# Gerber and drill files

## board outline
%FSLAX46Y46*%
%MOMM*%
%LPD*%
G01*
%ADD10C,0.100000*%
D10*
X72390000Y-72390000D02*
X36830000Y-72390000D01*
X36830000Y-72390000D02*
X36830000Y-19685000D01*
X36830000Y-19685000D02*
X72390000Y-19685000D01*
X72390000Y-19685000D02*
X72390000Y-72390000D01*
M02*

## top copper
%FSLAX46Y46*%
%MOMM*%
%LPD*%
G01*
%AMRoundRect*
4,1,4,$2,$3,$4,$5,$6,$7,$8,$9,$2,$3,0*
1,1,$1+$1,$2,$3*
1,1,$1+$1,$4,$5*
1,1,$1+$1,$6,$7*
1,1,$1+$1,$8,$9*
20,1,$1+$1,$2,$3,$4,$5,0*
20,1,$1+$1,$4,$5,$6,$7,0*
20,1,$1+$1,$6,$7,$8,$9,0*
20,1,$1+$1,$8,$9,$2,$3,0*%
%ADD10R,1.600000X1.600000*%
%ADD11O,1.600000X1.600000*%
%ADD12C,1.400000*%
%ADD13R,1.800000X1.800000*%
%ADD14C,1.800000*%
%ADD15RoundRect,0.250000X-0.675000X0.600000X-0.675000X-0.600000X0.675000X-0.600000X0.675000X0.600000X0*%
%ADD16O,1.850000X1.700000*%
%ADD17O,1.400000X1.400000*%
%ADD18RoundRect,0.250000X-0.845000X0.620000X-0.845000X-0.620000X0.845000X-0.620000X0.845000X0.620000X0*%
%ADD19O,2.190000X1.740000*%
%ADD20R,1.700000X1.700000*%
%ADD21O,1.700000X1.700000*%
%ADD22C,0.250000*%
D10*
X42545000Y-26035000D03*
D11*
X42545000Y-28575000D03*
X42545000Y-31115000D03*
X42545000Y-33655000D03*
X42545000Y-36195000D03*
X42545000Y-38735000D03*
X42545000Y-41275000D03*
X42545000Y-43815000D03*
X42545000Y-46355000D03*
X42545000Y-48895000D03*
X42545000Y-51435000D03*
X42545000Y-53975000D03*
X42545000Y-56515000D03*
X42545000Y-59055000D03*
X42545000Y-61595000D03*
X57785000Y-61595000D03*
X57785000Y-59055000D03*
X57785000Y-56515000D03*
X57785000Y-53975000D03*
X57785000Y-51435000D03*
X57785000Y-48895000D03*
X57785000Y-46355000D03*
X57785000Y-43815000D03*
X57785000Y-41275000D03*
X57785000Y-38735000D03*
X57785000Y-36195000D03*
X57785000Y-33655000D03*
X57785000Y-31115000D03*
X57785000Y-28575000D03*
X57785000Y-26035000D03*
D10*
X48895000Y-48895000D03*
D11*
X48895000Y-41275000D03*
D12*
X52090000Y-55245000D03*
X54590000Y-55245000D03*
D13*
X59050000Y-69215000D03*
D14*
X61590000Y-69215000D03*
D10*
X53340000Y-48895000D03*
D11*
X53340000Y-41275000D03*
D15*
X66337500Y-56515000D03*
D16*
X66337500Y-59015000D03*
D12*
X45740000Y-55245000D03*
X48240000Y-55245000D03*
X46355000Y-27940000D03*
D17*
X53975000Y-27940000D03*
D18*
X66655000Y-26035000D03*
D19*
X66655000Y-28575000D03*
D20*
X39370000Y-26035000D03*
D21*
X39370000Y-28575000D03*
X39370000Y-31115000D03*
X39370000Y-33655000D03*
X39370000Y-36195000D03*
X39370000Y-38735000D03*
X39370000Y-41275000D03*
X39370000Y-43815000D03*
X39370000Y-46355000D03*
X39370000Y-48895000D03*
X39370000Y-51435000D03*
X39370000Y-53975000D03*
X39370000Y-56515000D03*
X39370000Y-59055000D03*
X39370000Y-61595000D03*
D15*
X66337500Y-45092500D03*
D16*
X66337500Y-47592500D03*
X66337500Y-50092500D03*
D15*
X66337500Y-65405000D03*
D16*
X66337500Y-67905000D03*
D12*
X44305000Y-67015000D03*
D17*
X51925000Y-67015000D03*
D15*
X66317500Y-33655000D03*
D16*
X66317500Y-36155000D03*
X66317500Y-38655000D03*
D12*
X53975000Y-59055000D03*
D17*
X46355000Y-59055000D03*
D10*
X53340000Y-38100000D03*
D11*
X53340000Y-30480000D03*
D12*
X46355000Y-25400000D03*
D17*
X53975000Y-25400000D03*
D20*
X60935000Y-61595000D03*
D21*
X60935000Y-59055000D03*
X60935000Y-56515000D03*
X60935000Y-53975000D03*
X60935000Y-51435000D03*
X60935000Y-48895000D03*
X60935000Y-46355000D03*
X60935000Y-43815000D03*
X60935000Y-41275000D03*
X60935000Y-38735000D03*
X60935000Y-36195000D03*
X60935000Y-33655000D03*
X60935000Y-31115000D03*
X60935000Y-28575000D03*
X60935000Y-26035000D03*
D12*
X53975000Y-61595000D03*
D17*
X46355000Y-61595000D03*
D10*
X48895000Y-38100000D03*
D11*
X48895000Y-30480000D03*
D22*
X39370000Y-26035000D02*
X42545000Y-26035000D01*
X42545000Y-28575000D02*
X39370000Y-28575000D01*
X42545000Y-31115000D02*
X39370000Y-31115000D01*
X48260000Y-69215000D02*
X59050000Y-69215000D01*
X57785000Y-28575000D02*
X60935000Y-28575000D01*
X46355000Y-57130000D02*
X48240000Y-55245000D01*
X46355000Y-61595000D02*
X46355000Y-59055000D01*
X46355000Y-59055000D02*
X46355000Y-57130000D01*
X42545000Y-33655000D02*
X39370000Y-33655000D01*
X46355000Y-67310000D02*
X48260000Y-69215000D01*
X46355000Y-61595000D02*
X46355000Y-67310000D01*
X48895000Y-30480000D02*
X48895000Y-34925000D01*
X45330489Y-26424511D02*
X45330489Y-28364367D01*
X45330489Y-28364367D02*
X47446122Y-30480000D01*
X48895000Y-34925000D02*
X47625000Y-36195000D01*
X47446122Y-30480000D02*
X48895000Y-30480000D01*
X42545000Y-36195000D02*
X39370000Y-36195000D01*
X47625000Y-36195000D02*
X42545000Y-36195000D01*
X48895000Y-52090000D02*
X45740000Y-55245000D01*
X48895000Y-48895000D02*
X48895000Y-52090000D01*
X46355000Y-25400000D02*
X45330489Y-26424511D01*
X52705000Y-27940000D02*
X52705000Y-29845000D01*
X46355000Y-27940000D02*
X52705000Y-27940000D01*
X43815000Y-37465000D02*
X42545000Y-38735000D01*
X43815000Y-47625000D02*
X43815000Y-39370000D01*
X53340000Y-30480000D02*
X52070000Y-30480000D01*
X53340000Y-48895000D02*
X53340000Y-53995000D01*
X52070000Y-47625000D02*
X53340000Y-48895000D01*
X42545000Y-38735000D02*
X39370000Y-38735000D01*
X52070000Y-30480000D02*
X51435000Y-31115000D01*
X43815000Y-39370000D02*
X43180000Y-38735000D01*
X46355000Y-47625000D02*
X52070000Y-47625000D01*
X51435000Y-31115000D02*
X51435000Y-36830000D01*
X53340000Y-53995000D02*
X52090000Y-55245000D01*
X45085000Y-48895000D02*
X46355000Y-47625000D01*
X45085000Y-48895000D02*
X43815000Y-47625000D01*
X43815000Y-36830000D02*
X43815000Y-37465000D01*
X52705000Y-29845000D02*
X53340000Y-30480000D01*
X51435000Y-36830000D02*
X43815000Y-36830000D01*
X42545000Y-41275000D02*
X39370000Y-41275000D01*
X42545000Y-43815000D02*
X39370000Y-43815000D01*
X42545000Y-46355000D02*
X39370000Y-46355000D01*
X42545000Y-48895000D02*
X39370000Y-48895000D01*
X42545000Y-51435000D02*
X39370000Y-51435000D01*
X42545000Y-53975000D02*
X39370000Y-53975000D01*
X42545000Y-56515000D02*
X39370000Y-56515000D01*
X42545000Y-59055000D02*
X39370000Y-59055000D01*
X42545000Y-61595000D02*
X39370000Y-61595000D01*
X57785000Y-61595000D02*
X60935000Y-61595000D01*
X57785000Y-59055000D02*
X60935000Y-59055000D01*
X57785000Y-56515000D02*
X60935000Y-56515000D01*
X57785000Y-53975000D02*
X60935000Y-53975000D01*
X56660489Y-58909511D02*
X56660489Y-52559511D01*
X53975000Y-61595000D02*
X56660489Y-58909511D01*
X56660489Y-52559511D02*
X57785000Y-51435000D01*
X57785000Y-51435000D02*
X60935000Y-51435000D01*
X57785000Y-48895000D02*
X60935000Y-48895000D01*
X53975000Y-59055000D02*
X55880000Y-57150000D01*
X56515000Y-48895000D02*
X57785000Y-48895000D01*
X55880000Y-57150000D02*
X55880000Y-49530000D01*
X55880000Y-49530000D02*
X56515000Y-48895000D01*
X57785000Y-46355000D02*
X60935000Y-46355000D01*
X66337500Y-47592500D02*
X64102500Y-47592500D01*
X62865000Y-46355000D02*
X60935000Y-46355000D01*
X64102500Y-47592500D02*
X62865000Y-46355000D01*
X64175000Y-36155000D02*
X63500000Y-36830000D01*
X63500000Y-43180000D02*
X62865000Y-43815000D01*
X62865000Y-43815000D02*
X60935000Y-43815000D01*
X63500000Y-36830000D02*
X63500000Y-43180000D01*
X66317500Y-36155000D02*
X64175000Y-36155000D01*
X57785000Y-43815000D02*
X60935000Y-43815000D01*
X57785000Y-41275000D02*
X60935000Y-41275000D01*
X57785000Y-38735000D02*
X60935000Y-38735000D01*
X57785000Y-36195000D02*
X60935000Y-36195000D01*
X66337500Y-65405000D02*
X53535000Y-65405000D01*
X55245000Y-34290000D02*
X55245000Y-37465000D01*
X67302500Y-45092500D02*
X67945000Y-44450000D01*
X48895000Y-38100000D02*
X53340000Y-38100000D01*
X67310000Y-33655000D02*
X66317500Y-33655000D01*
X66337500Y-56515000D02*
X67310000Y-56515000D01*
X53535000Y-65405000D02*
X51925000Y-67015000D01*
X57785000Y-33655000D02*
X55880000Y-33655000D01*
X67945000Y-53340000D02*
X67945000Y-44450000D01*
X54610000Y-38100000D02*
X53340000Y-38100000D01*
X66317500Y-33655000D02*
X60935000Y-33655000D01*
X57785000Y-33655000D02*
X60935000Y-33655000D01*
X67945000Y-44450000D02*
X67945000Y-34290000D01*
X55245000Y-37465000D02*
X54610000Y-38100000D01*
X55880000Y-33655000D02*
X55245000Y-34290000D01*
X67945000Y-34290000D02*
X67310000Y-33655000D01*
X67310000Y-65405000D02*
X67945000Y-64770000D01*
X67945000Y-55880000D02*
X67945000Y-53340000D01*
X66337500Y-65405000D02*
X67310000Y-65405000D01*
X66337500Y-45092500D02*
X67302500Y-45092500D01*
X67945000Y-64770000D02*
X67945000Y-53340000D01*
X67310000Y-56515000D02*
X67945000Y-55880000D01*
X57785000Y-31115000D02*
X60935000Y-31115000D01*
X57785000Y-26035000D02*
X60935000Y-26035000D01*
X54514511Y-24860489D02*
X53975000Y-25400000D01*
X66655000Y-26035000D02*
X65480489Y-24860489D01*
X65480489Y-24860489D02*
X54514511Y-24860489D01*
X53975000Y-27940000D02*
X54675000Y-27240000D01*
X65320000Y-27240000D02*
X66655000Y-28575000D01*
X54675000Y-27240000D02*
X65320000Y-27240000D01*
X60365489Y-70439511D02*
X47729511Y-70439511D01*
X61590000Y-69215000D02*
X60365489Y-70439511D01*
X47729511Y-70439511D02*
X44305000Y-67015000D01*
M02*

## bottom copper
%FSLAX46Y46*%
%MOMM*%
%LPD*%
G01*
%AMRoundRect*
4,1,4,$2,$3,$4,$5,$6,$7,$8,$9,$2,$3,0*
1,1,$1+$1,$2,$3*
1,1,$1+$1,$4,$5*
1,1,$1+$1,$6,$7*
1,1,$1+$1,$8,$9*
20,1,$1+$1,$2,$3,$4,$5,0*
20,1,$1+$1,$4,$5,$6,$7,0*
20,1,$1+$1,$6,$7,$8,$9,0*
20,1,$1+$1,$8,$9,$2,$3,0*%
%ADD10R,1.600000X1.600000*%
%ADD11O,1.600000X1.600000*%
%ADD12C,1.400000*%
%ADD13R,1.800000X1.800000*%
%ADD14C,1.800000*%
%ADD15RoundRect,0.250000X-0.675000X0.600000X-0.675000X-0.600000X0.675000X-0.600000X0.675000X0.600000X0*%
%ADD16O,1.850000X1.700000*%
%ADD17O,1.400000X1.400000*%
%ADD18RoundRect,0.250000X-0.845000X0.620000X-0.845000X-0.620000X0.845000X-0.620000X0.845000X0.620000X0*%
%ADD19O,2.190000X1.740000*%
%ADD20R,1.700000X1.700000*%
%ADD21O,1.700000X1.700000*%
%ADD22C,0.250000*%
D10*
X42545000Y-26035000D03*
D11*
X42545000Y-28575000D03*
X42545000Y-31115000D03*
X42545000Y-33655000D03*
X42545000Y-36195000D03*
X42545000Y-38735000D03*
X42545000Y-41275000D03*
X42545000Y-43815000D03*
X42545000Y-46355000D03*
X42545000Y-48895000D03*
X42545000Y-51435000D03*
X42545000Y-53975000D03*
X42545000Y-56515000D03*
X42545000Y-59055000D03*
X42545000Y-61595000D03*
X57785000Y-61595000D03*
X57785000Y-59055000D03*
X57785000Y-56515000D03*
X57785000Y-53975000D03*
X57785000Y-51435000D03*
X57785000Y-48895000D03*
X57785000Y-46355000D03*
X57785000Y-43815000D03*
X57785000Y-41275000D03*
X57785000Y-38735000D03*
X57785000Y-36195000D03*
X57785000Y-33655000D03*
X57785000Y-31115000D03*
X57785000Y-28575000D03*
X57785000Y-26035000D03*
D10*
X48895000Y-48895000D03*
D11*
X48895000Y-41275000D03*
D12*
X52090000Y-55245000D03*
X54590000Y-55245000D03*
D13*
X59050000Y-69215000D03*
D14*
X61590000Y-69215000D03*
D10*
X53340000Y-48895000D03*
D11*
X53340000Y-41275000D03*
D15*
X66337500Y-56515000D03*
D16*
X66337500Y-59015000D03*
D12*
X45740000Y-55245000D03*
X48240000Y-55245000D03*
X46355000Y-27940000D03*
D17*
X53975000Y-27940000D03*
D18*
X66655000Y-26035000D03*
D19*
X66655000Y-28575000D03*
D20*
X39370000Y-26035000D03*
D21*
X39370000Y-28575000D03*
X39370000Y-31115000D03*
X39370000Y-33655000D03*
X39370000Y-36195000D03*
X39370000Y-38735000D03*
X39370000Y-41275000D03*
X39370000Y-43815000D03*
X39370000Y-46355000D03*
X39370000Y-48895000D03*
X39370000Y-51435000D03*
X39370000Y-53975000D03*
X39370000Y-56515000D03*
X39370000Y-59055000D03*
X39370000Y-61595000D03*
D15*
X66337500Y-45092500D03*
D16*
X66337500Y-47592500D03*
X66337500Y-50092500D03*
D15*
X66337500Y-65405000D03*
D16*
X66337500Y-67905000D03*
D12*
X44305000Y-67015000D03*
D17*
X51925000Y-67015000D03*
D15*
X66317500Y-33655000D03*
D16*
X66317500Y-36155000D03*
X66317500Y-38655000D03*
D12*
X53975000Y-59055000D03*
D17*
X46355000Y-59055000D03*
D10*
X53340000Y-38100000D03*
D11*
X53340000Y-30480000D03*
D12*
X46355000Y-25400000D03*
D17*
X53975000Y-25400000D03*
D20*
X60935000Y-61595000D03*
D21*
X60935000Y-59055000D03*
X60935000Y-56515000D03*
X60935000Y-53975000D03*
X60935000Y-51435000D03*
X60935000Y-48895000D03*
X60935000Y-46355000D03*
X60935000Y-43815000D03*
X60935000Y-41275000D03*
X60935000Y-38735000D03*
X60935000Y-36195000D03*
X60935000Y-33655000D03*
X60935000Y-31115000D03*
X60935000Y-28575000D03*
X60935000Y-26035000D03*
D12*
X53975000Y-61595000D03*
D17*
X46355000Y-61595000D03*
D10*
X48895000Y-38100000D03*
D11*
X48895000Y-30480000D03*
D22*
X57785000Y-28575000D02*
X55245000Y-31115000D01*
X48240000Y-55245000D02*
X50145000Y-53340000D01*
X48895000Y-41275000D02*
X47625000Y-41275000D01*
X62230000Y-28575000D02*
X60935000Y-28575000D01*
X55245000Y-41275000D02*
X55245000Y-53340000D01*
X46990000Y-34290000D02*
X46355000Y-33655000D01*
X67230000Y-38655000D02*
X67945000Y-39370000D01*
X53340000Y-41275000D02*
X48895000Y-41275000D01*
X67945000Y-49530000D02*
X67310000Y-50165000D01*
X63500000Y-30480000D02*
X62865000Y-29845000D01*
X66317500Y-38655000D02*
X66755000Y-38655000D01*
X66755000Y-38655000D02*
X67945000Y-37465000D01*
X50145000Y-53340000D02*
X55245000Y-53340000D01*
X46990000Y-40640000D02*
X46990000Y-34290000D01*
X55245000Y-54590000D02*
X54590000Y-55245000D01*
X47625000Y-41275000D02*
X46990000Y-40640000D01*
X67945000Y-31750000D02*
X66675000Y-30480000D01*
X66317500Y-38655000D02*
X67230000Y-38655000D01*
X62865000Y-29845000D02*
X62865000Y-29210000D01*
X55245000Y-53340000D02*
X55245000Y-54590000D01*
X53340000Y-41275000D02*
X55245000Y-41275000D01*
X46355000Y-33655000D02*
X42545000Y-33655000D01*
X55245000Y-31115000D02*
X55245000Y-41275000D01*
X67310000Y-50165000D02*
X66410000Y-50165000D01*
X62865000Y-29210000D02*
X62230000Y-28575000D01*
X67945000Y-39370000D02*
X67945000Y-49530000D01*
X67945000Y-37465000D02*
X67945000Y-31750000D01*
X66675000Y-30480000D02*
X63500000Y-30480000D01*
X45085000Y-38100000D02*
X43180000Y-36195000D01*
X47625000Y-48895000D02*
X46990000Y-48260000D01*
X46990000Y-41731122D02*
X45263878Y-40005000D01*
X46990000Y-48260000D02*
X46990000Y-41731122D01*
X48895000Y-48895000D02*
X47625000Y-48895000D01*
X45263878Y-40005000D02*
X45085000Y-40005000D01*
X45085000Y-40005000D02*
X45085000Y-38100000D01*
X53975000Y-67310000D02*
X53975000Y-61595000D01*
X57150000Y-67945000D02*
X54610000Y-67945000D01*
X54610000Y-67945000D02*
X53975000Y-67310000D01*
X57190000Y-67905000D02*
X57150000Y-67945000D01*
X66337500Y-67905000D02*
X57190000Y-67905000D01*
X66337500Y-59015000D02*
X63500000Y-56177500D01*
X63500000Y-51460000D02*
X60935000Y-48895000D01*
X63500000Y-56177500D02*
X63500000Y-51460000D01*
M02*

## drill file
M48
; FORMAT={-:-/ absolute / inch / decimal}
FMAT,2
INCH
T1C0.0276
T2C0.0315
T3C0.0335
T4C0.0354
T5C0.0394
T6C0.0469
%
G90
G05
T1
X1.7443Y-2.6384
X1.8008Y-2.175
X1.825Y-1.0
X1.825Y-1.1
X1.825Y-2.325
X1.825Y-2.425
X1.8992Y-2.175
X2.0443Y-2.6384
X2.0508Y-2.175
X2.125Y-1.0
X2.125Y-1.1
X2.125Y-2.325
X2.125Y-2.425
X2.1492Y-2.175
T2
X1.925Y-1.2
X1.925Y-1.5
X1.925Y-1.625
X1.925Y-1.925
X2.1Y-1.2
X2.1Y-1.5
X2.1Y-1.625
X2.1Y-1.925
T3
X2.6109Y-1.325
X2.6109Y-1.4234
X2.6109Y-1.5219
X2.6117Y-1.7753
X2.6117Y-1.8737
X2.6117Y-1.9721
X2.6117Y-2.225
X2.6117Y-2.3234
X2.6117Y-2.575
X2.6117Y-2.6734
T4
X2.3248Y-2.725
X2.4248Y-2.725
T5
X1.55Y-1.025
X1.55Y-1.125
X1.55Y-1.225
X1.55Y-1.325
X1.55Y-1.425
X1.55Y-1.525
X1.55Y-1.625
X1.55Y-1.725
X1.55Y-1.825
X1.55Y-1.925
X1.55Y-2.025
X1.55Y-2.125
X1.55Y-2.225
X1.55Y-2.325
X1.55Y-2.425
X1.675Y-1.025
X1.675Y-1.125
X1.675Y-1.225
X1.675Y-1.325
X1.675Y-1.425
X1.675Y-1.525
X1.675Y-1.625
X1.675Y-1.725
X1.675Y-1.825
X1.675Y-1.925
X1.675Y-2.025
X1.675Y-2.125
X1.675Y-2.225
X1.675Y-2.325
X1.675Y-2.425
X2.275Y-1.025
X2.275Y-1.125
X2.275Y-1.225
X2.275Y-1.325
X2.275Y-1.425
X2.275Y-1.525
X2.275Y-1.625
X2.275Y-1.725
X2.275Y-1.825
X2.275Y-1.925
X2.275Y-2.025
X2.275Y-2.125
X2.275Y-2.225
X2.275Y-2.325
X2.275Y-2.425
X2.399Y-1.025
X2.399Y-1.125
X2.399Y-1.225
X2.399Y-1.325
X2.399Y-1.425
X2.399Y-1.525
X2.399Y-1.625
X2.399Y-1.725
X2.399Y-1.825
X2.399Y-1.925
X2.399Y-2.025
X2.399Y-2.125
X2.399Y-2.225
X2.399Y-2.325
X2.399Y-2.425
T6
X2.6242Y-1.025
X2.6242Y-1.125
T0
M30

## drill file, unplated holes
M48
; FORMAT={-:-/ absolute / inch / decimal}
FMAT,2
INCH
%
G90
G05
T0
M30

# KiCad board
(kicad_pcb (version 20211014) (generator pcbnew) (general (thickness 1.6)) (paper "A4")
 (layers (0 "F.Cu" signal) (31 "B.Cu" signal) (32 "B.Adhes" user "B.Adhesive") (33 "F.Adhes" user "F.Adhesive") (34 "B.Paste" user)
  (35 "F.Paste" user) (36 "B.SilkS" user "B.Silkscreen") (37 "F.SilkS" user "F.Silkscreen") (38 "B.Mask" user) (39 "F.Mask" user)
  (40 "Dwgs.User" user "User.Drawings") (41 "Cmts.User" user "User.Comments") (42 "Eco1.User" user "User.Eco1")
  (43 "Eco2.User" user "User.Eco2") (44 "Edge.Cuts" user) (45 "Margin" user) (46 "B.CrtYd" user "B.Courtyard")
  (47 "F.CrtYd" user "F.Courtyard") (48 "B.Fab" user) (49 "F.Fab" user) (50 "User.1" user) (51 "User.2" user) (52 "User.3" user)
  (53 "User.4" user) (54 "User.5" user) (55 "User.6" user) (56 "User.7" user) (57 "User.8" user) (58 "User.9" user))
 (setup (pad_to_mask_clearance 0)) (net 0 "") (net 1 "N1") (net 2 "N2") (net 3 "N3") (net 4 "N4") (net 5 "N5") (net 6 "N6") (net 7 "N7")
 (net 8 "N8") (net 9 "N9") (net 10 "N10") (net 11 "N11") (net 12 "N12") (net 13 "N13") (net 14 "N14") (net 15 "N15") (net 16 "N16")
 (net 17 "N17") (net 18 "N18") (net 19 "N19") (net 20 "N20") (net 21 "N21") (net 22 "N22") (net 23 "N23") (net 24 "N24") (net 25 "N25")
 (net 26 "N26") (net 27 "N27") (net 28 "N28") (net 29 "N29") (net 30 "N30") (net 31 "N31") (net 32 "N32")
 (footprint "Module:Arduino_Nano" (layer "F.Cu") (at 42.545 26.035)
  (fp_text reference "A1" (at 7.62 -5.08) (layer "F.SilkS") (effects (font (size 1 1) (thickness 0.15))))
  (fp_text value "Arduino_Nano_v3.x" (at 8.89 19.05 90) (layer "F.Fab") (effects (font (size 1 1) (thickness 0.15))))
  (pad "1" thru_hole rect (at 0 0) (size 1.6 1.6) (drill 1) (layers *.Cu *.Mask) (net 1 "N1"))
  (pad "2" thru_hole oval (at 0 2.54) (size 1.6 1.6) (drill 1) (layers *.Cu *.Mask) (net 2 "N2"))
  (pad "3" thru_hole oval (at 0 5.08) (size 1.6 1.6) (drill 1) (layers *.Cu *.Mask) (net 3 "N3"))
  (pad "4" thru_hole oval (at 0 7.62) (size 1.6 1.6) (drill 1) (layers *.Cu *.Mask) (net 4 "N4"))
  (pad "5" thru_hole oval (at 0 10.16) (size 1.6 1.6) (drill 1) (layers *.Cu *.Mask) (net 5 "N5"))
  (pad "6" thru_hole oval (at 0 12.7) (size 1.6 1.6) (drill 1) (layers *.Cu *.Mask) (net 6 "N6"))
  (pad "7" thru_hole oval (at 0 15.24) (size 1.6 1.6) (drill 1) (layers *.Cu *.Mask) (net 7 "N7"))
  (pad "8" thru_hole oval (at 0 17.78) (size 1.6 1.6) (drill 1) (layers *.Cu *.Mask) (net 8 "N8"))
  (pad "9" thru_hole oval (at 0 20.32) (size 1.6 1.6) (drill 1) (layers *.Cu *.Mask) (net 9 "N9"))
  (pad "10" thru_hole oval (at 0 22.86) (size 1.6 1.6) (drill 1) (layers *.Cu *.Mask) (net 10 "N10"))
  (pad "11" thru_hole oval (at 0 25.4) (size 1.6 1.6) (drill 1) (layers *.Cu *.Mask) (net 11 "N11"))
  (pad "12" thru_hole oval (at 0 27.94) (size 1.6 1.6) (drill 1) (layers *.Cu *.Mask) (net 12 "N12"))
  (pad "13" thru_hole oval (at 0 30.48) (size 1.6 1.6) (drill 1) (layers *.Cu *.Mask) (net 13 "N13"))
  (pad "14" thru_hole oval (at 0 33.02) (size 1.6 1.6) (drill 1) (layers *.Cu *.Mask) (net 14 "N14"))
  (pad "15" thru_hole oval (at 0 35.56) (size 1.6 1.6) (drill 1) (layers *.Cu *.Mask) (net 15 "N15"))
  (pad "16" thru_hole oval (at 15.24 35.56) (size 1.6 1.6) (drill 1) (layers *.Cu *.Mask) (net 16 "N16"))
  (pad "17" thru_hole oval (at 15.24 33.02) (size 1.6 1.6) (drill 1) (layers *.Cu *.Mask) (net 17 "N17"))
  (pad "18" thru_hole oval (at 15.24 30.48) (size 1.6 1.6) (drill 1) (layers *.Cu *.Mask) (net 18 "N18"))
  (pad "19" thru_hole oval (at 15.24 27.94) (size 1.6 1.6) (drill 1) (layers *.Cu *.Mask) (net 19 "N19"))
  (pad "20" thru_hole oval (at 15.24 25.4) (size 1.6 1.6) (drill 1) (layers *.Cu *.Mask) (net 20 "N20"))
  (pad "21" thru_hole oval (at 15.24 22.86) (size 1.6 1.6) (drill 1) (layers *.Cu *.Mask) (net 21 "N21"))
  (pad "22" thru_hole oval (at 15.24 20.32) (size 1.6 1.6) (drill 1) (layers *.Cu *.Mask) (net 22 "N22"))
  (pad "23" thru_hole oval (at 15.24 17.78) (size 1.6 1.6) (drill 1) (layers *.Cu *.Mask) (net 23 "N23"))
  (pad "24" thru_hole oval (at 15.24 15.24) (size 1.6 1.6) (drill 1) (layers *.Cu *.Mask) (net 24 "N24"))
  (pad "25" thru_hole oval (at 15.24 12.7) (size 1.6 1.6) (drill 1) (layers *.Cu *.Mask) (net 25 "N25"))
  (pad "26" thru_hole oval (at 15.24 10.16) (size 1.6 1.6) (drill 1) (layers *.Cu *.Mask) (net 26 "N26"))
  (pad "27" thru_hole oval (at 15.24 7.62) (size 1.6 1.6) (drill 1) (layers *.Cu *.Mask) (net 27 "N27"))
  (pad "28" thru_hole oval (at 15.24 5.08) (size 1.6 1.6) (drill 1) (layers *.Cu *.Mask) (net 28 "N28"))
  (pad "29" thru_hole oval (at 15.24 2.54) (size 1.6 1.6) (drill 1) (layers *.Cu *.Mask) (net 4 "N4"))
  (pad "30" thru_hole oval (at 15.24 0) (size 1.6 1.6) (drill 1) (layers *.Cu *.Mask) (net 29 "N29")))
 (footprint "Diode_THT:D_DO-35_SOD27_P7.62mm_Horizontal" (layer "F.Cu") (at 48.895 48.895 90)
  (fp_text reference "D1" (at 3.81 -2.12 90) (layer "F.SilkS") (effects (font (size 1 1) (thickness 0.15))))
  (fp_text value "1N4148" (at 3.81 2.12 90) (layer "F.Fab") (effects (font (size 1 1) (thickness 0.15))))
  (pad "1" thru_hole rect (at 0 0 90) (size 1.6 1.6) (drill 0.8) (layers *.Cu *.Mask) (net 5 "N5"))
  (pad "2" thru_hole oval (at 7.62 0 90) (size 1.6 1.6) (drill 0.8) (layers *.Cu *.Mask) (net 4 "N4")))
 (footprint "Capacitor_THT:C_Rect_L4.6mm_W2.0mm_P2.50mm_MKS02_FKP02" (layer "F.Cu") (at 52.09 55.245)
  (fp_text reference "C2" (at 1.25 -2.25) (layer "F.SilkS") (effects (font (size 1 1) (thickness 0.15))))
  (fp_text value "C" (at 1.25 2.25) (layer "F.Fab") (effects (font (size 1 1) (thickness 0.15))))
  (pad "1" thru_hole circle (at 0 0) (size 1.4 1.4) (drill 0.7) (layers *.Cu *.Mask) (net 6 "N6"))
  (pad "2" thru_hole circle (at 2.5 0) (size 1.4 1.4) (drill 0.7) (layers *.Cu *.Mask) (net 4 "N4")))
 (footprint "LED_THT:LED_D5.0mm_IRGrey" (layer "F.Cu") (at 59.05 69.215)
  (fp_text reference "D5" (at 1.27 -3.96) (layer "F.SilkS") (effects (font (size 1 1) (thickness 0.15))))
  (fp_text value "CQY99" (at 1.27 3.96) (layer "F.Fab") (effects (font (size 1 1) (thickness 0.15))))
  (pad "1" thru_hole rect (at 0 0) (size 1.8 1.8) (drill 0.9) (layers *.Cu *.Mask) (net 4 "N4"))
  (pad "2" thru_hole circle (at 2.54 0) (size 1.8 1.8) (drill 0.9) (layers *.Cu *.Mask) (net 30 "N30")))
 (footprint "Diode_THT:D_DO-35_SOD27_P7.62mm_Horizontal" (layer "F.Cu") (at 53.34 48.895 90)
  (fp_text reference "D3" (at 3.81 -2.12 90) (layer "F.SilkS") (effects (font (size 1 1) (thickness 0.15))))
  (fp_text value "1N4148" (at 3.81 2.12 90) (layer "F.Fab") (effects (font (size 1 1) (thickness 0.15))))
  (pad "1" thru_hole rect (at 0 0 90) (size 1.6 1.6) (drill 0.8) (layers *.Cu *.Mask) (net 6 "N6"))
  (pad "2" thru_hole oval (at 7.62 0 90) (size 1.6 1.6) (drill 0.8) (layers *.Cu *.Mask) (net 4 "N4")))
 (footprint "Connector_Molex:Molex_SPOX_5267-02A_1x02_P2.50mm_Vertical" (layer "F.Cu") (at 66.3375 56.515 -90)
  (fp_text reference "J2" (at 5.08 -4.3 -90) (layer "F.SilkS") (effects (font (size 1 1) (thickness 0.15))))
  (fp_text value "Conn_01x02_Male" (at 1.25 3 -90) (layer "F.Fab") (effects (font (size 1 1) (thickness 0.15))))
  (pad "1" thru_hole roundrect (at 0 0 270) (size 1.7 1.85) (drill 0.85) (layers *.Cu *.Mask) (roundrect_rratio 0.1470588235) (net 27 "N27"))
  (pad "2" thru_hole oval (at 2.5 0 270) (size 1.7 1.85) (drill 0.85) (layers *.Cu *.Mask) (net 21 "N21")))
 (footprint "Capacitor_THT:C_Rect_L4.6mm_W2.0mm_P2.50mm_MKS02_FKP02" (layer "F.Cu") (at 45.74 55.245)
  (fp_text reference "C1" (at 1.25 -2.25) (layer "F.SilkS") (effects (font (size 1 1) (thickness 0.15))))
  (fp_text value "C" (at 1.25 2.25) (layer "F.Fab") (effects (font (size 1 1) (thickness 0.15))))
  (pad "1" thru_hole circle (at 0 0) (size 1.4 1.4) (drill 0.7) (layers *.Cu *.Mask) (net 5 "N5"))
  (pad "2" thru_hole circle (at 2.5 0) (size 1.4 1.4) (drill 0.7) (layers *.Cu *.Mask) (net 4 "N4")))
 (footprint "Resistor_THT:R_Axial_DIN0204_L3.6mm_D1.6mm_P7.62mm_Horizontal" (layer "F.Cu") (at 46.355 27.94)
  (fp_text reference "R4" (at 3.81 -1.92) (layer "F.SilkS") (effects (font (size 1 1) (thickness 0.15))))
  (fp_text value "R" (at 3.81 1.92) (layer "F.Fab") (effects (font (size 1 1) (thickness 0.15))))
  (pad "1" thru_hole circle (at 0 0) (size 1.4 1.4) (drill 0.7) (layers *.Cu *.Mask) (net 6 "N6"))
  (pad "2" thru_hole oval (at 7.62 0) (size 1.4 1.4) (drill 0.7) (layers *.Cu *.Mask) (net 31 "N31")))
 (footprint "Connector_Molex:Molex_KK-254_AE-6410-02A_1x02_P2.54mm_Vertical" (layer "F.Cu") (at 66.655 26.035 -90)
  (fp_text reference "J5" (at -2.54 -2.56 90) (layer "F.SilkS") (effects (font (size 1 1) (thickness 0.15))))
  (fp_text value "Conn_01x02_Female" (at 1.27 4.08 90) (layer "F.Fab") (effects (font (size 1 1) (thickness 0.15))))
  (pad "1" thru_hole roundrect (at 0 0 270) (size 1.74 2.19) (drill 1.19) (layers *.Cu *.Mask) (roundrect_rratio 0.1436781609)
   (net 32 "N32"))
  (pad "2" thru_hole oval (at 2.54 0 270) (size 1.74 2.19) (drill 1.19) (layers *.Cu *.Mask) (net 31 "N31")))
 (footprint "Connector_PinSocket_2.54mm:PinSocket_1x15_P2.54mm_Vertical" (layer "F.Cu") (at 39.37 26.035)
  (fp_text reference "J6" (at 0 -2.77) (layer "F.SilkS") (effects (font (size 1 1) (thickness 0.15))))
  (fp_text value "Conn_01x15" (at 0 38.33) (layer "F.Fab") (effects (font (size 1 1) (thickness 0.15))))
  (pad "1" thru_hole rect (at 0 0) (size 1.7 1.7) (drill 1) (layers *.Cu *.Mask) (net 1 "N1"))
  (pad "2" thru_hole oval (at 0 2.54) (size 1.7 1.7) (drill 1) (layers *.Cu *.Mask) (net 2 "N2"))
  (pad "3" thru_hole oval (at 0 5.08) (size 1.7 1.7) (drill 1) (layers *.Cu *.Mask) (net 3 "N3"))
  (pad "4" thru_hole oval (at 0 7.62) (size 1.7 1.7) (drill 1) (layers *.Cu *.Mask) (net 4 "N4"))
  (pad "5" thru_hole oval (at 0 10.16) (size 1.7 1.7) (drill 1) (layers *.Cu *.Mask) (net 5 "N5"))
  (pad "6" thru_hole oval (at 0 12.7) (size 1.7 1.7) (drill 1) (layers *.Cu *.Mask) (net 6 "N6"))
  (pad "7" thru_hole oval (at 0 15.24) (size 1.7 1.7) (drill 1) (layers *.Cu *.Mask) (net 7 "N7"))
  (pad "8" thru_hole oval (at 0 17.78) (size 1.7 1.7) (drill 1) (layers *.Cu *.Mask) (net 8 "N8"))
  (pad "9" thru_hole oval (at 0 20.32) (size 1.7 1.7) (drill 1) (layers *.Cu *.Mask) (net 9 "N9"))
  (pad "10" thru_hole oval (at 0 22.86) (size 1.7 1.7) (drill 1) (layers *.Cu *.Mask) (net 10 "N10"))
  (pad "11" thru_hole oval (at 0 25.4) (size 1.7 1.7) (drill 1) (layers *.Cu *.Mask) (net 11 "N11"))
  (pad "12" thru_hole oval (at 0 27.94) (size 1.7 1.7) (drill 1) (layers *.Cu *.Mask) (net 12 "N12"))
  (pad "13" thru_hole oval (at 0 30.48) (size 1.7 1.7) (drill 1) (layers *.Cu *.Mask) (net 13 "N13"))
  (pad "14" thru_hole oval (at 0 33.02) (size 1.7 1.7) (drill 1) (layers *.Cu *.Mask) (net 14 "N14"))
  (pad "15" thru_hole oval (at 0 35.56) (size 1.7 1.7) (drill 1) (layers *.Cu *.Mask) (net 15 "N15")))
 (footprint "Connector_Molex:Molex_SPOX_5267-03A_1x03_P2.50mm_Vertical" (layer "F.Cu") (at 66.3375 45.0925 -90)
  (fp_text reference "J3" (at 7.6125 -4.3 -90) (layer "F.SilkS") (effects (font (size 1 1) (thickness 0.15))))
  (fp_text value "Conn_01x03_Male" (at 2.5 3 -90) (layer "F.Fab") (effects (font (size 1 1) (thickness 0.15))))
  (pad "1" thru_hole roundrect (at 0 0 270) (size 1.7 1.85) (drill 0.85) (layers *.Cu *.Mask) (roundrect_rratio 0.1470588235) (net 27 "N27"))
  (pad "2" thru_hole oval (at 2.5 0 270) (size 1.7 1.85) (drill 0.85) (layers *.Cu *.Mask) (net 22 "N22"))
  (pad "3" thru_hole oval (at 5 0 270) (size 1.7 1.85) (drill 0.85) (layers *.Cu *.Mask) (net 4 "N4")))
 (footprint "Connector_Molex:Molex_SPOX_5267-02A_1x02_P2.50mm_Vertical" (layer "F.Cu") (at 66.3375 65.405 -90)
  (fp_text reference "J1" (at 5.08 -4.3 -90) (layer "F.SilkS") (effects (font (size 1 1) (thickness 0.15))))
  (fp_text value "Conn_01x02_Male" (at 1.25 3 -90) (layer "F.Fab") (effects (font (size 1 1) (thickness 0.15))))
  (pad "1" thru_hole roundrect (at 0 0 270) (size 1.7 1.85) (drill 0.85) (layers *.Cu *.Mask) (roundrect_rratio 0.1470588235) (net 27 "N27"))
  (pad "2" thru_hole oval (at 2.5 0 270) (size 1.7 1.85) (drill 0.85) (layers *.Cu *.Mask) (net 20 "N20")))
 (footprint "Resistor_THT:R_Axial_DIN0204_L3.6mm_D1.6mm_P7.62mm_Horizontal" (layer "F.Cu") (at 44.305 67.015)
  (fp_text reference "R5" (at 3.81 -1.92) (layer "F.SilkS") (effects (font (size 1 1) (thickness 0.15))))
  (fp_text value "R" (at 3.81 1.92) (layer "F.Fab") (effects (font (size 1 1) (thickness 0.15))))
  (pad "1" thru_hole circle (at 0 0) (size 1.4 1.4) (drill 0.7) (layers *.Cu *.Mask) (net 30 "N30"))
  (pad "2" thru_hole oval (at 7.62 0) (size 1.4 1.4) (drill 0.7) (layers *.Cu *.Mask) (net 27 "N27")))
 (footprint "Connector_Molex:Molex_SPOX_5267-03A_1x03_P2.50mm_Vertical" (layer "F.Cu") (at 66.3175 33.655 -90)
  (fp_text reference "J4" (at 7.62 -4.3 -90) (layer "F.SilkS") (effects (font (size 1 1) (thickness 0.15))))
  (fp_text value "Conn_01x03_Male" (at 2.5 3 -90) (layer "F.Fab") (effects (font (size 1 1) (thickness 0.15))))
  (pad "1" thru_hole roundrect (at 0 0 270) (size 1.7 1.85) (drill 0.85) (layers *.Cu *.Mask) (roundrect_rratio 0.1470588235) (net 27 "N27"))
  (pad "2" thru_hole oval (at 2.5 0 270) (size 1.7 1.85) (drill 0.85) (layers *.Cu *.Mask) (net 23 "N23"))
  (pad "3" thru_hole oval (at 5 0 270) (size 1.7 1.85) (drill 0.85) (layers *.Cu *.Mask) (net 4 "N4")))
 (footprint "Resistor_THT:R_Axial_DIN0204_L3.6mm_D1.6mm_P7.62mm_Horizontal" (layer "F.Cu") (at 53.975 59.055 180)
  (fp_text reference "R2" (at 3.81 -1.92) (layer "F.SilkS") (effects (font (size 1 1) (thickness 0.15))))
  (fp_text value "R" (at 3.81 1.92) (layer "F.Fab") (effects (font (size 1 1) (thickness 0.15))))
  (pad "1" thru_hole circle (at 0 0 180) (size 1.4 1.4) (drill 0.7) (layers *.Cu *.Mask) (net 21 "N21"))
  (pad "2" thru_hole oval (at 7.62 0 180) (size 1.4 1.4) (drill 0.7) (layers *.Cu *.Mask) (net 4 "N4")))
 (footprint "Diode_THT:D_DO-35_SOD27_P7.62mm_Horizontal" (layer "F.Cu") (at 53.34 38.1 90)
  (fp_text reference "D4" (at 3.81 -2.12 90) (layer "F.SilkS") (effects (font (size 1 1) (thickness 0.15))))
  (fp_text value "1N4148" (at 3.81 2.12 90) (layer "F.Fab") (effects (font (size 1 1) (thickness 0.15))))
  (pad "1" thru_hole rect (at 0 0 90) (size 1.6 1.6) (drill 0.8) (layers *.Cu *.Mask) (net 27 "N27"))
  (pad "2" thru_hole oval (at 7.62 0 90) (size 1.6 1.6) (drill 0.8) (layers *.Cu *.Mask) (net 6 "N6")))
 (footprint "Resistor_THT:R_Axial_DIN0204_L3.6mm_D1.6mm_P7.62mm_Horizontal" (layer "F.Cu") (at 46.355 25.4)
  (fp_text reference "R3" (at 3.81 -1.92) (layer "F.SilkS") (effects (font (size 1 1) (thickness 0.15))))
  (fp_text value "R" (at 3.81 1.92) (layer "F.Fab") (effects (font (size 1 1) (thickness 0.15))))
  (pad "1" thru_hole circle (at 0 0) (size 1.4 1.4) (drill 0.7) (layers *.Cu *.Mask) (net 5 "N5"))
  (pad "2" thru_hole oval (at 7.62 0) (size 1.4 1.4) (drill 0.7) (layers *.Cu *.Mask) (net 32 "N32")))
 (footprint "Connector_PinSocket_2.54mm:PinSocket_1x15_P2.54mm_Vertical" (layer "F.Cu") (at 60.935 61.595 180)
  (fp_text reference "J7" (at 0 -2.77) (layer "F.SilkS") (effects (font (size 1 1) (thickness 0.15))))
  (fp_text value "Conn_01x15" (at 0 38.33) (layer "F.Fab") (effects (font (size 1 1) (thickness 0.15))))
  (pad "1" thru_hole rect (at 0 0 180) (size 1.7 1.7) (drill 1) (layers *.Cu *.Mask) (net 16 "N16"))
  (pad "2" thru_hole oval (at 0 2.54 180) (size 1.7 1.7) (drill 1) (layers *.Cu *.Mask) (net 17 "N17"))
  (pad "3" thru_hole oval (at 0 5.08 180) (size 1.7 1.7) (drill 1) (layers *.Cu *.Mask) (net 18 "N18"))
  (pad "4" thru_hole oval (at 0 7.62 180) (size 1.7 1.7) (drill 1) (layers *.Cu *.Mask) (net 19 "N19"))
  (pad "5" thru_hole oval (at 0 10.16 180) (size 1.7 1.7) (drill 1) (layers *.Cu *.Mask) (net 20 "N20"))
  (pad "6" thru_hole oval (at 0 12.7 180) (size 1.7 1.7) (drill 1) (layers *.Cu *.Mask) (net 21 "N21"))
  (pad "7" thru_hole oval (at 0 15.24 180) (size 1.7 1.7) (drill 1) (layers *.Cu *.Mask) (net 22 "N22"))
  (pad "8" thru_hole oval (at 0 17.78 180) (size 1.7 1.7) (drill 1) (layers *.Cu *.Mask) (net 23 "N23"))
  (pad "9" thru_hole oval (at 0 20.32 180) (size 1.7 1.7) (drill 1) (layers *.Cu *.Mask) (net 24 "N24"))
  (pad "10" thru_hole oval (at 0 22.86 180) (size 1.7 1.7) (drill 1) (layers *.Cu *.Mask) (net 25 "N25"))
  (pad "11" thru_hole oval (at 0 25.4 180) (size 1.7 1.7) (drill 1) (layers *.Cu *.Mask) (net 26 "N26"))
  (pad "12" thru_hole oval (at 0 27.94 180) (size 1.7 1.7) (drill 1) (layers *.Cu *.Mask) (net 27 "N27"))
  (pad "13" thru_hole oval (at 0 30.48 180) (size 1.7 1.7) (drill 1) (layers *.Cu *.Mask) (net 28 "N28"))
  (pad "14" thru_hole oval (at 0 33.02 180) (size 1.7 1.7) (drill 1) (layers *.Cu *.Mask) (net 4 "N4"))
  (pad "15" thru_hole oval (at 0 35.56 180) (size 1.7 1.7) (drill 1) (layers *.Cu *.Mask) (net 29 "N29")))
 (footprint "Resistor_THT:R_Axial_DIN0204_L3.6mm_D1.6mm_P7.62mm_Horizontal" (layer "F.Cu") (at 53.975 61.595 180)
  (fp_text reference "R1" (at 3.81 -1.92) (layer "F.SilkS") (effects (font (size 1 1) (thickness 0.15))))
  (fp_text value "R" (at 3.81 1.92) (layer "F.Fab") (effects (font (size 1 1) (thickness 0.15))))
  (pad "1" thru_hole circle (at 0 0 180) (size 1.4 1.4) (drill 0.7) (layers *.Cu *.Mask) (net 20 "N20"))
  (pad "2" thru_hole oval (at 7.62 0 180) (size 1.4 1.4) (drill 0.7) (layers *.Cu *.Mask) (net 4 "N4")))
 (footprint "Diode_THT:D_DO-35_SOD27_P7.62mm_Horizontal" (layer "F.Cu") (at 48.895 38.1 90)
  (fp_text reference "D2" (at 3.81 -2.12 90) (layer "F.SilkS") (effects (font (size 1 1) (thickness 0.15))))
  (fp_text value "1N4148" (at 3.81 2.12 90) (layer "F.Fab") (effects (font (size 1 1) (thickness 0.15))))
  (pad "1" thru_hole rect (at 0 0 90) (size 1.6 1.6) (drill 0.8) (layers *.Cu *.Mask) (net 27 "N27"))
  (pad "2" thru_hole oval (at 7.62 0 90) (size 1.6 1.6) (drill 0.8) (layers *.Cu *.Mask) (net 5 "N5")))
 (gr_rect (start 72.39 72.39) (end 36.83 19.685) (layer "Edge.Cuts") (width 0.1) (fill none))
 (segment (start 39.37 26.035) (end 42.545 26.035) (width 0.25) (layer "F.Cu") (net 1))
 (segment (start 42.545 28.575) (end 39.37 28.575) (width 0.25) (layer "F.Cu") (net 2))
 (segment (start 42.545 31.115) (end 39.37 31.115) (width 0.25) (layer "F.Cu") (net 3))
 (segment (start 48.26 69.215) (end 59.05 69.215) (width 0.25) (layer "F.Cu") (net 4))
 (segment (start 57.785 28.575) (end 60.935 28.575) (width 0.25) (layer "F.Cu") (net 4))
 (segment (start 46.355 57.13) (end 48.24 55.245) (width 0.25) (layer "F.Cu") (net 4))
 (segment (start 46.355 61.595) (end 46.355 59.055) (width 0.25) (layer "F.Cu") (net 4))
 (segment (start 46.355 59.055) (end 46.355 57.13) (width 0.25) (layer "F.Cu") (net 4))
 (segment (start 42.545 33.655) (end 39.37 33.655) (width 0.25) (layer "F.Cu") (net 4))
 (segment (start 46.355 67.31) (end 48.26 69.215) (width 0.25) (layer "F.Cu") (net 4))
 (segment (start 46.355 61.595) (end 46.355 67.31) (width 0.25) (layer "F.Cu") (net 4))
 (segment (start 57.785 28.575) (end 55.245 31.115) (width 0.25) (layer "B.Cu") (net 4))
 (segment (start 48.24 55.245) (end 50.145 53.34) (width 0.25) (layer "B.Cu") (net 4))
 (segment (start 48.895 41.275) (end 47.625 41.275) (width 0.25) (layer "B.Cu") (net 4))
 (segment (start 62.23 28.575) (end 60.935 28.575) (width 0.25) (layer "B.Cu") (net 4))
 (segment (start 55.245 41.275) (end 55.245 53.34) (width 0.25) (layer "B.Cu") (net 4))
 (segment (start 46.99 34.29) (end 46.355 33.655) (width 0.25) (layer "B.Cu") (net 4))
 (segment (start 67.23 38.655) (end 67.945 39.37) (width 0.25) (layer "B.Cu") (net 4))
 (segment (start 53.34 41.275) (end 48.895 41.275) (width 0.25) (layer "B.Cu") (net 4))
 (segment (start 67.945 49.53) (end 67.31 50.165) (width 0.25) (layer "B.Cu") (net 4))
 (segment (start 63.5 30.48) (end 62.865 29.845) (width 0.25) (layer "B.Cu") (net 4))
 (segment (start 66.3175 38.655) (end 66.755 38.655) (width 0.25) (layer "B.Cu") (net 4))
 (segment (start 66.755 38.655) (end 67.945 37.465) (width 0.25) (layer "B.Cu") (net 4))
 (segment (start 50.145 53.34) (end 55.245 53.34) (width 0.25) (layer "B.Cu") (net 4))
 (segment (start 46.99 40.64) (end 46.99 34.29) (width 0.25) (layer "B.Cu") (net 4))
 (segment (start 55.245 54.59) (end 54.59 55.245) (width 0.25) (layer "B.Cu") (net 4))
 (segment (start 47.625 41.275) (end 46.99 40.64) (width 0.25) (layer "B.Cu") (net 4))
 (segment (start 67.945 31.75) (end 66.675 30.48) (width 0.25) (layer "B.Cu") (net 4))
 (segment (start 66.3175 38.655) (end 67.23 38.655) (width 0.25) (layer "B.Cu") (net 4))
 (segment (start 62.865 29.845) (end 62.865 29.21) (width 0.25) (layer "B.Cu") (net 4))
 (segment (start 55.245 53.34) (end 55.245 54.59) (width 0.25) (layer "B.Cu") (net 4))
 (segment (start 53.34 41.275) (end 55.245 41.275) (width 0.25) (layer "B.Cu") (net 4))
 (segment (start 46.355 33.655) (end 42.545 33.655) (width 0.25) (layer "B.Cu") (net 4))
 (segment (start 55.245 31.115) (end 55.245 41.275) (width 0.25) (layer "B.Cu") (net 4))
 (segment (start 67.31 50.165) (end 66.41 50.165) (width 0.25) (layer "B.Cu") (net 4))
 (segment (start 62.865 29.21) (end 62.23 28.575) (width 0.25) (layer "B.Cu") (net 4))
 (segment (start 67.945 39.37) (end 67.945 49.53) (width 0.25) (layer "B.Cu") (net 4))
 (segment (start 67.945 37.465) (end 67.945 31.75) (width 0.25) (layer "B.Cu") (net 4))
 (segment (start 66.675 30.48) (end 63.5 30.48) (width 0.25) (layer "B.Cu") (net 4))
 (segment (start 48.895 30.48) (end 48.895 34.925) (width 0.25) (layer "F.Cu") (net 5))
 (segment (start 45.330489 26.424511) (end 45.330489 28.364367) (width 0.25) (layer "F.Cu") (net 5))
 (segment (start 45.330489 28.364367) (end 47.446122 30.48) (width 0.25) (layer "F.Cu") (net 5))
 (segment (start 48.895 34.925) (end 47.625 36.195) (width 0.25) (layer "F.Cu") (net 5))
 (segment (start 47.446122 30.48) (end 48.895 30.48) (width 0.25) (layer "F.Cu") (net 5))
 (segment (start 42.545 36.195) (end 39.37 36.195) (width 0.25) (layer "F.Cu") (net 5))
 (segment (start 47.625 36.195) (end 42.545 36.195) (width 0.25) (layer "F.Cu") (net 5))
 (segment (start 48.895 52.09) (end 45.74 55.245) (width 0.25) (layer "F.Cu") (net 5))
 (segment (start 48.895 48.895) (end 48.895 52.09) (width 0.25) (layer "F.Cu") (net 5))
 (segment (start 46.355 25.4) (end 45.330489 26.424511) (width 0.25) (layer "F.Cu") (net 5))
 (segment (start 45.085 38.1) (end 43.18 36.195) (width 0.25) (layer "B.Cu") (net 5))
 (segment (start 47.625 48.895) (end 46.99 48.26) (width 0.25) (layer "B.Cu") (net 5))
 (segment (start 46.99 41.731122) (end 45.263878 40.005) (width 0.25) (layer "B.Cu") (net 5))
 (segment (start 46.99 48.26) (end 46.99 41.731122) (width 0.25) (layer "B.Cu") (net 5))
 (segment (start 48.895 48.895) (end 47.625 48.895) (width 0.25) (layer "B.Cu") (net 5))
 (segment (start 45.263878 40.005) (end 45.085 40.005) (width 0.25) (layer "B.Cu") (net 5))
 (segment (start 45.085 40.005) (end 45.085 38.1) (width 0.25) (layer "B.Cu") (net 5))
 (segment (start 52.705 27.94) (end 52.705 29.845) (width 0.25) (layer "F.Cu") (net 6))
 (segment (start 46.355 27.94) (end 52.705 27.94) (width 0.25) (layer "F.Cu") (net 6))
 (segment (start 43.815 37.465) (end 42.545 38.735) (width 0.25) (layer "F.Cu") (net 6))
 (segment (start 43.815 47.625) (end 43.815 39.37) (width 0.25) (layer "F.Cu") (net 6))
 (segment (start 53.34 30.48) (end 52.07 30.48) (width 0.25) (layer "F.Cu") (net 6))
 (segment (start 53.34 48.895) (end 53.34 53.995) (width 0.25) (layer "F.Cu") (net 6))
 (segment (start 52.07 47.625) (end 53.34 48.895) (width 0.25) (layer "F.Cu") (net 6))
 (segment (start 42.545 38.735) (end 39.37 38.735) (width 0.25) (layer "F.Cu") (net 6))
 (segment (start 52.07 30.48) (end 51.435 31.115) (width 0.25) (layer "F.Cu") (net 6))
 (segment (start 43.815 39.37) (end 43.18 38.735) (width 0.25) (layer "F.Cu") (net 6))
 (segment (start 46.355 47.625) (end 52.07 47.625) (width 0.25) (layer "F.Cu") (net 6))
 (segment (start 51.435 31.115) (end 51.435 36.83) (width 0.25) (layer "F.Cu") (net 6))
 (segment (start 53.34 53.995) (end 52.09 55.245) (width 0.25) (layer "F.Cu") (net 6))
 (segment (start 45.085 48.895) (end 46.355 47.625) (width 0.25) (layer "F.Cu") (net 6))
 (segment (start 45.085 48.895) (end 43.815 47.625) (width 0.25) (layer "F.Cu") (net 6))
 (segment (start 43.815 36.83) (end 43.815 37.465) (width 0.25) (layer "F.Cu") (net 6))
 (segment (start 52.705 29.845) (end 53.34 30.48) (width 0.25) (layer "F.Cu") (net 6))
 (segment (start 51.435 36.83) (end 43.815 36.83) (width 0.25) (layer "F.Cu") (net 6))
 (segment (start 42.545 41.275) (end 39.37 41.275) (width 0.25) (layer "F.Cu") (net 7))
 (segment (start 42.545 43.815) (end 39.37 43.815) (width 0.25) (layer "F.Cu") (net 8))
 (segment (start 42.545 46.355) (end 39.37 46.355) (width 0.25) (layer "F.Cu") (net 9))
 (segment (start 42.545 48.895) (end 39.37 48.895) (width 0.25) (layer "F.Cu") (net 10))
 (segment (start 42.545 51.435) (end 39.37 51.435) (width 0.25) (layer "F.Cu") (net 11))
 (segment (start 42.545 53.975) (end 39.37 53.975) (width 0.25) (layer "F.Cu") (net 12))
 (segment (start 42.545 56.515) (end 39.37 56.515) (width 0.25) (layer "F.Cu") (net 13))
 (segment (start 42.545 59.055) (end 39.37 59.055) (width 0.25) (layer "F.Cu") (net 14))
 (segment (start 42.545 61.595) (end 39.37 61.595) (width 0.25) (layer "F.Cu") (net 15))
 (segment (start 57.785 61.595) (end 60.935 61.595) (width 0.25) (layer "F.Cu") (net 16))
 (segment (start 57.785 59.055) (end 60.935 59.055) (width 0.25) (layer "F.Cu") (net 17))
 (segment (start 57.785 56.515) (end 60.935 56.515) (width 0.25) (layer "F.Cu") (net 18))
 (segment (start 57.785 53.975) (end 60.935 53.975) (width 0.25) (layer "F.Cu") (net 19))
 (segment (start 56.660489 58.909511) (end 56.660489 52.559511) (width 0.25) (layer "F.Cu") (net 20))
 (segment (start 53.975 61.595) (end 56.660489 58.909511) (width 0.25) (layer "F.Cu") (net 20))
 (segment (start 56.660489 52.559511) (end 57.785 51.435) (width 0.25) (layer "F.Cu") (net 20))
 (segment (start 57.785 51.435) (end 60.935 51.435) (width 0.25) (layer "F.Cu") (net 20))
 (segment (start 53.975 67.31) (end 53.975 61.595) (width 0.25) (layer "B.Cu") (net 20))
 (segment (start 57.15 67.945) (end 54.61 67.945) (width 0.25) (layer "B.Cu") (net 20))
 (segment (start 54.61 67.945) (end 53.975 67.31) (width 0.25) (layer "B.Cu") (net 20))
 (segment (start 57.19 67.905) (end 57.15 67.945) (width 0.25) (layer "B.Cu") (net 20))
 (segment (start 66.3375 67.905) (end 57.19 67.905) (width 0.25) (layer "B.Cu") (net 20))
 (segment (start 57.785 48.895) (end 60.935 48.895) (width 0.25) (layer "F.Cu") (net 21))
 (segment (start 53.975 59.055) (end 55.88 57.15) (width 0.25) (layer "F.Cu") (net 21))
 (segment (start 56.515 48.895) (end 57.785 48.895) (width 0.25) (layer "F.Cu") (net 21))
 (segment (start 55.88 57.15) (end 55.88 49.53) (width 0.25) (layer "F.Cu") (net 21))
 (segment (start 55.88 49.53) (end 56.515 48.895) (width 0.25) (layer "F.Cu") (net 21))
 (segment (start 66.3375 59.015) (end 63.5 56.1775) (width 0.25) (layer "B.Cu") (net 21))
 (segment (start 63.5 51.46) (end 60.935 48.895) (width 0.25) (layer "B.Cu") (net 21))
 (segment (start 63.5 56.1775) (end 63.5 51.46) (width 0.25) (layer "B.Cu") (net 21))
 (segment (start 57.785 46.355) (end 60.935 46.355) (width 0.25) (layer "F.Cu") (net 22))
 (segment (start 66.3375 47.5925) (end 64.1025 47.5925) (width 0.25) (layer "F.Cu") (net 22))
 (segment (start 62.865 46.355) (end 60.935 46.355) (width 0.25) (layer "F.Cu") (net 22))
 (segment (start 64.1025 47.5925) (end 62.865 46.355) (width 0.25) (layer "F.Cu") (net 22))
 (segment (start 64.175 36.155) (end 63.5 36.83) (width 0.25) (layer "F.Cu") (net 23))
 (segment (start 63.5 43.18) (end 62.865 43.815) (width 0.25) (layer "F.Cu") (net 23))
 (segment (start 62.865 43.815) (end 60.935 43.815) (width 0.25) (layer "F.Cu") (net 23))
 (segment (start 63.5 36.83) (end 63.5 43.18) (width 0.25) (layer "F.Cu") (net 23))
 (segment (start 66.3175 36.155) (end 64.175 36.155) (width 0.25) (layer "F.Cu") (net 23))
 (segment (start 57.785 43.815) (end 60.935 43.815) (width 0.25) (layer "F.Cu") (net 23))
 (segment (start 57.785 41.275) (end 60.935 41.275) (width 0.25) (layer "F.Cu") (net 24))
 (segment (start 57.785 38.735) (end 60.935 38.735) (width 0.25) (layer "F.Cu") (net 25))
 (segment (start 57.785 36.195) (end 60.935 36.195) (width 0.25) (layer "F.Cu") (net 26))
 (segment (start 66.3375 65.405) (end 53.535 65.405) (width 0.25) (layer "F.Cu") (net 27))
 (segment (start 55.245 34.29) (end 55.245 37.465) (width 0.25) (layer "F.Cu") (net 27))
 (segment (start 67.3025 45.0925) (end 67.945 44.45) (width 0.25) (layer "F.Cu") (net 27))
 (segment (start 48.895 38.1) (end 53.34 38.1) (width 0.25) (layer "F.Cu") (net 27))
 (segment (start 67.31 33.655) (end 66.3175 33.655) (width 0.25) (layer "F.Cu") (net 27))
 (segment (start 66.3375 56.515) (end 67.31 56.515) (width 0.25) (layer "F.Cu") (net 27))
 (segment (start 53.535 65.405) (end 51.925 67.015) (width 0.25) (layer "F.Cu") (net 27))
 (segment (start 57.785 33.655) (end 55.88 33.655) (width 0.25) (layer "F.Cu") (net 27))
 (segment (start 67.945 53.34) (end 67.945 44.45) (width 0.25) (layer "F.Cu") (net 27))
 (segment (start 54.61 38.1) (end 53.34 38.1) (width 0.25) (layer "F.Cu") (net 27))
 (segment (start 66.3175 33.655) (end 60.935 33.655) (width 0.25) (layer "F.Cu") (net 27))
 (segment (start 57.785 33.655) (end 60.935 33.655) (width 0.25) (layer "F.Cu") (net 27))
 (segment (start 67.945 44.45) (end 67.945 34.29) (width 0.25) (layer "F.Cu") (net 27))
 (segment (start 55.245 37.465) (end 54.61 38.1) (width 0.25) (layer "F.Cu") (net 27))
 (segment (start 55.88 33.655) (end 55.245 34.29) (width 0.25) (layer "F.Cu") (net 27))
 (segment (start 67.945 34.29) (end 67.31 33.655) (width 0.25) (layer "F.Cu") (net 27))
 (segment (start 67.31 65.405) (end 67.945 64.77) (width 0.25) (layer "F.Cu") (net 27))
 (segment (start 67.945 55.88) (end 67.945 53.34) (width 0.25) (layer "F.Cu") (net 27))
 (segment (start 66.3375 65.405) (end 67.31 65.405) (width 0.25) (layer "F.Cu") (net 27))
 (segment (start 66.3375 45.0925) (end 67.3025 45.0925) (width 0.25) (layer "F.Cu") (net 27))
 (segment (start 67.945 64.77) (end 67.945 53.34) (width 0.25) (layer "F.Cu") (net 27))
 (segment (start 67.31 56.515) (end 67.945 55.88) (width 0.25) (layer "F.Cu") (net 27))
 (segment (start 57.785 31.115) (end 60.935 31.115) (width 0.25) (layer "F.Cu") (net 28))
 (segment (start 57.785 26.035) (end 60.935 26.035) (width 0.25) (layer "F.Cu") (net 29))
 (segment (start 54.514511 24.860489) (end 53.975 25.4) (width 0.25) (layer "F.Cu") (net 32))
 (segment (start 66.655 26.035) (end 65.480489 24.860489) (width 0.25) (layer "F.Cu") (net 32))
 (segment (start 65.480489 24.860489) (end 54.514511 24.860489) (width 0.25) (layer "F.Cu") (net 32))
 (segment (start 53.975 27.94) (end 54.675 27.24) (width 0.25) (layer "F.Cu") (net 31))
 (segment (start 65.32 27.24) (end 66.655 28.575) (width 0.25) (layer "F.Cu") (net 31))
 (segment (start 54.675 27.24) (end 65.32 27.24) (width 0.25) (layer "F.Cu") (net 31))
 (segment (start 60.365489 70.439511) (end 47.729511 70.439511) (width 0.25) (layer "F.Cu") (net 30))
 (segment (start 61.59 69.215) (end 60.365489 70.439511) (width 0.25) (layer "F.Cu") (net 30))
 (segment (start 47.729511 70.439511) (end 44.305 67.015) (width 0.25) (layer "F.Cu") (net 30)))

